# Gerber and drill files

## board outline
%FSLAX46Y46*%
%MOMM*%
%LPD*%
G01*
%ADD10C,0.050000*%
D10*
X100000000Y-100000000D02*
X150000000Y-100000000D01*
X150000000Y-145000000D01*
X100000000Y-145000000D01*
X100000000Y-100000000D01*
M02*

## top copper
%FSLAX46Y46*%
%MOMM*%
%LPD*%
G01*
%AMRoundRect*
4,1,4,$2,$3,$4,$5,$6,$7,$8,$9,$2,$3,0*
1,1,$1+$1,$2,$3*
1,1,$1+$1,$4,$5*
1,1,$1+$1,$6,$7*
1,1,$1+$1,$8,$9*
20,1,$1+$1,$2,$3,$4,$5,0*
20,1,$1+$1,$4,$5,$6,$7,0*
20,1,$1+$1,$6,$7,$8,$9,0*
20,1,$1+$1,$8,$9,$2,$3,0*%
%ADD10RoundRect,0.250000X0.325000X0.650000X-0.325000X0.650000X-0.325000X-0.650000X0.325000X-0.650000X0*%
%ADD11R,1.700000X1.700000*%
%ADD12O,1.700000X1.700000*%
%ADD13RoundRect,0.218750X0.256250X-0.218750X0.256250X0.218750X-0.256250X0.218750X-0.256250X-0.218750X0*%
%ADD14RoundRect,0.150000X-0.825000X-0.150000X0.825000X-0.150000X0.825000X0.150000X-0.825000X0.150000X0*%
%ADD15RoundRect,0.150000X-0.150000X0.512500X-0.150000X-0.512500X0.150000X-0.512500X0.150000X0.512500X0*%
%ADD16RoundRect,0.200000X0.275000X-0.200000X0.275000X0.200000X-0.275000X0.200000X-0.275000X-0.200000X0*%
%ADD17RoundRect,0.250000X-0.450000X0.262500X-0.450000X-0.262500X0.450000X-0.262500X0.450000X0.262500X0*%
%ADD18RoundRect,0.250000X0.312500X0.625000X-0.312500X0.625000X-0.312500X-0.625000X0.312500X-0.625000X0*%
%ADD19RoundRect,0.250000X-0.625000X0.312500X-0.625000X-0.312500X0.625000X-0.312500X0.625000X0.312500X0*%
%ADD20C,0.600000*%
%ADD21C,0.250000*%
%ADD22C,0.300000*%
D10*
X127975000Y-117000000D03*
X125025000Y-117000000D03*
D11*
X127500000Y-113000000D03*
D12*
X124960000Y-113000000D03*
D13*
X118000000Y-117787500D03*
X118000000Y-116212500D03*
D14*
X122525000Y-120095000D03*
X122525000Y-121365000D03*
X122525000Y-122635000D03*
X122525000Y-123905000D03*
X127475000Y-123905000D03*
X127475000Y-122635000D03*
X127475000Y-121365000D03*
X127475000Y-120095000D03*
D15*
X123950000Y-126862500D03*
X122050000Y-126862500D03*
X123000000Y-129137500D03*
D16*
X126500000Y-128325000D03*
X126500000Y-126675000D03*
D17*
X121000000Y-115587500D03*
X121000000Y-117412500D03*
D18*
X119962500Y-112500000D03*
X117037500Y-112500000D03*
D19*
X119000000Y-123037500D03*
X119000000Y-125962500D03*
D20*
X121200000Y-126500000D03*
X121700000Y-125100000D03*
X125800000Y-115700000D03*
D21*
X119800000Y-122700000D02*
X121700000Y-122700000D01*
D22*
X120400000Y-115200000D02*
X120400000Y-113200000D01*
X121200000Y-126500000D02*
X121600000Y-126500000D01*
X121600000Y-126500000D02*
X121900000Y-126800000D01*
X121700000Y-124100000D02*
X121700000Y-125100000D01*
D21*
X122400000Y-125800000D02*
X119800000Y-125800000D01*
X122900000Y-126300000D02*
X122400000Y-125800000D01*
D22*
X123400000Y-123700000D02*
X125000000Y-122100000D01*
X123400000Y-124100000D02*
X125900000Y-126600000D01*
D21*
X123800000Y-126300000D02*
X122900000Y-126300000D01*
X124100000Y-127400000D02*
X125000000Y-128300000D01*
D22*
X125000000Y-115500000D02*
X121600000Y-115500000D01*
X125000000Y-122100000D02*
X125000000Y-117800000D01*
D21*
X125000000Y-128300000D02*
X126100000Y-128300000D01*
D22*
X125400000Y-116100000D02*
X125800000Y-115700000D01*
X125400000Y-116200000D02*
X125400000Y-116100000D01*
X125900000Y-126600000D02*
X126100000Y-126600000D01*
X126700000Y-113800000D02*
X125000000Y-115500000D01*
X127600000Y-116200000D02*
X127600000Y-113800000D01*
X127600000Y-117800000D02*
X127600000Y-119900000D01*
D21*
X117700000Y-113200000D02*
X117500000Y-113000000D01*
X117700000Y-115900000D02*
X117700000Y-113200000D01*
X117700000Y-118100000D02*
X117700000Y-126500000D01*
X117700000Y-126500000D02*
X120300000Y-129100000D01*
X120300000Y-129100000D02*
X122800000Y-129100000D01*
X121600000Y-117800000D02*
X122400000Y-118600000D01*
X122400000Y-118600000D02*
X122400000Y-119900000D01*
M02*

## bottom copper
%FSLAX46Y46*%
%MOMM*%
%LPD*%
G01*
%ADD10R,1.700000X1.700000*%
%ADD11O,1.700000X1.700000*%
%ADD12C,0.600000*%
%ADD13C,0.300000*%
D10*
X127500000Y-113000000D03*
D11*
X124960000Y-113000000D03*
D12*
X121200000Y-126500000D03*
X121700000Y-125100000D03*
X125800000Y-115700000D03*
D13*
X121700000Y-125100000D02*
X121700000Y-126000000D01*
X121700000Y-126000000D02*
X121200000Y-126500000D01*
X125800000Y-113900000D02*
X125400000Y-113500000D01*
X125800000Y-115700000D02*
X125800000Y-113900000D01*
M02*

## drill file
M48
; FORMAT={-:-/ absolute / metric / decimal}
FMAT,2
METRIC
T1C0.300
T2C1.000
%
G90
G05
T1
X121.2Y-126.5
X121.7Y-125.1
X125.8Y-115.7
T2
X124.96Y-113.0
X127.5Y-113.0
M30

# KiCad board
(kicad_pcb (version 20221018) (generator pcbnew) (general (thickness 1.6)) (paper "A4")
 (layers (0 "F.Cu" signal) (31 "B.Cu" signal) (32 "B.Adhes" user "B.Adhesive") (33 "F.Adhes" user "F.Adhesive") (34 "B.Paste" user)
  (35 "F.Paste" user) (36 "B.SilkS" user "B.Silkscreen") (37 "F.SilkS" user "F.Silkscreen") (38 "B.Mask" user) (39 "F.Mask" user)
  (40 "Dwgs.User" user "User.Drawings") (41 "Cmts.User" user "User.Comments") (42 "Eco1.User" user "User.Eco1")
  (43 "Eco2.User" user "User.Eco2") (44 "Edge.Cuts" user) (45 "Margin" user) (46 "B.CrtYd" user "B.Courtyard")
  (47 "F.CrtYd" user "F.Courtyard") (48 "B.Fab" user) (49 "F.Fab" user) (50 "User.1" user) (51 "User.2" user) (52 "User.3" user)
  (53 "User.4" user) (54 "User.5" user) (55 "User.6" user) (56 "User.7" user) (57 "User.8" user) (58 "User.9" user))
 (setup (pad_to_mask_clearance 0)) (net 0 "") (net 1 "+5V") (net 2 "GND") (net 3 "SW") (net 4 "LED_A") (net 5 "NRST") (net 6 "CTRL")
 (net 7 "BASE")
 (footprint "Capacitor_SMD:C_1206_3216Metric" (layer "F.Cu") (at 126.5 117 180)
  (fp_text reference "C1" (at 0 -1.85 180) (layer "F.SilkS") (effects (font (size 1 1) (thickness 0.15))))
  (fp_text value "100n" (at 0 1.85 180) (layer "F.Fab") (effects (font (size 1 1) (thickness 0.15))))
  (pad "1" smd roundrect (at -1.475 0 180) (size 1.15 1.8) (layers "F.Cu" "F.Paste" "F.Mask") (roundrect_rratio 0.217391) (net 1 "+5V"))
  (pad "2" smd roundrect (at 1.475 0 180) (size 1.15 1.8) (layers "F.Cu" "F.Paste" "F.Mask") (roundrect_rratio 0.217391) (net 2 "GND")))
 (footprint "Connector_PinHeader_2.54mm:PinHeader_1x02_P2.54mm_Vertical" (layer "F.Cu") (at 127.5 113 -90)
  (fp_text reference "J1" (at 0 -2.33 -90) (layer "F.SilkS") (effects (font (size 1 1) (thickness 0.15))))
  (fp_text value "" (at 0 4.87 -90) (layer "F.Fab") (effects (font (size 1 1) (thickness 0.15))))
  (pad "1" thru_hole rect (at 0 0 270) (size 1.7 1.7) (drill 1) (layers "*.Cu" "*.Mask") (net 1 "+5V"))
  (pad "2" thru_hole oval (at 0 2.54 270) (size 1.7 1.7) (drill 1) (layers "*.Cu" "*.Mask") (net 2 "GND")))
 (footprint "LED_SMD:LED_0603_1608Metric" (layer "F.Cu") (at 118 117 90)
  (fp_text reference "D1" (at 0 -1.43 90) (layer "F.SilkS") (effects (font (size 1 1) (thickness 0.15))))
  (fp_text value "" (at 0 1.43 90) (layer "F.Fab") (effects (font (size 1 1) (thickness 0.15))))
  (pad "1" smd roundrect (at -0.7875 0 90) (size 0.875 0.95) (layers "F.Cu" "F.Paste" "F.Mask") (roundrect_rratio 0.25) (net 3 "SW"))
  (pad "2" smd roundrect (at 0.7875 0 90) (size 0.875 0.95) (layers "F.Cu" "F.Paste" "F.Mask") (roundrect_rratio 0.25) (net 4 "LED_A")))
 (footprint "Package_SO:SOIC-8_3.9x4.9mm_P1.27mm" (layer "F.Cu") (at 125 122)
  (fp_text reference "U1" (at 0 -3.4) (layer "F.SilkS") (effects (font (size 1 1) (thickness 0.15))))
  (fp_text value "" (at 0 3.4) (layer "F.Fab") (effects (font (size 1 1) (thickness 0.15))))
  (pad "1" smd roundrect (at -2.475 -1.905) (size 1.95 0.6) (layers "F.Cu" "F.Paste" "F.Mask") (roundrect_rratio 0.25) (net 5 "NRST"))
  (pad "2" smd roundrect (at -2.475 -0.635) (size 1.95 0.6) (layers "F.Cu" "F.Paste" "F.Mask") (roundrect_rratio 0.25))
  (pad "3" smd roundrect (at -2.475 0.635) (size 1.95 0.6) (layers "F.Cu" "F.Paste" "F.Mask") (roundrect_rratio 0.25) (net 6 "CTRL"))
  (pad "4" smd roundrect (at -2.475 1.905) (size 1.95 0.6) (layers "F.Cu" "F.Paste" "F.Mask") (roundrect_rratio 0.25) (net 2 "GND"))
  (pad "5" smd roundrect (at 2.475 1.905) (size 1.95 0.6) (layers "F.Cu" "F.Paste" "F.Mask") (roundrect_rratio 0.25))
  (pad "6" smd roundrect (at 2.475 0.635) (size 1.95 0.6) (layers "F.Cu" "F.Paste" "F.Mask") (roundrect_rratio 0.25))
  (pad "7" smd roundrect (at 2.475 -0.635) (size 1.95 0.6) (layers "F.Cu" "F.Paste" "F.Mask") (roundrect_rratio 0.25))
  (pad "8" smd roundrect (at 2.475 -1.905) (size 1.95 0.6) (layers "F.Cu" "F.Paste" "F.Mask") (roundrect_rratio 0.25) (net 1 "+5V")))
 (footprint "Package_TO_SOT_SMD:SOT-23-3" (layer "F.Cu") (at 123 128 -90)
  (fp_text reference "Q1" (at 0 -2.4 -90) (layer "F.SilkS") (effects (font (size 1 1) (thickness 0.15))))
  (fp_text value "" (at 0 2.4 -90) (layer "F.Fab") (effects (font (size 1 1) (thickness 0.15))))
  (pad "1" smd roundrect (at -1.1375 -0.95 270) (size 1.325 0.6) (layers "F.Cu" "F.Paste" "F.Mask") (roundrect_rratio 0.25) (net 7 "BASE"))
  (pad "2" smd roundrect (at -1.1375 0.95 270) (size 1.325 0.6) (layers "F.Cu" "F.Paste" "F.Mask") (roundrect_rratio 0.25) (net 2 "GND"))
  (pad "3" smd roundrect (at 1.1375 0 270) (size 1.325 0.6) (layers "F.Cu" "F.Paste" "F.Mask") (roundrect_rratio 0.25) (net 3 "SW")))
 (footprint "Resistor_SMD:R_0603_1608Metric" (layer "F.Cu") (at 126.5 127.5 90)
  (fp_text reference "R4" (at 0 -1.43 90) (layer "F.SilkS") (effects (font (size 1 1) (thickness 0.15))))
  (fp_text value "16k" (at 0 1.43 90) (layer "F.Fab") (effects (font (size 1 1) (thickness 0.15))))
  (pad "1" smd roundrect (at -0.825 0 90) (size 0.8 0.95) (layers "F.Cu" "F.Paste" "F.Mask") (roundrect_rratio 0.25) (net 7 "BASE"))
  (pad "2" smd roundrect (at 0.825 0 90) (size 0.8 0.95) (layers "F.Cu" "F.Paste" "F.Mask") (roundrect_rratio 0.25) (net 2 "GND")))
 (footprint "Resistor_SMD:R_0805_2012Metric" (layer "F.Cu") (at 121 116.5 -90)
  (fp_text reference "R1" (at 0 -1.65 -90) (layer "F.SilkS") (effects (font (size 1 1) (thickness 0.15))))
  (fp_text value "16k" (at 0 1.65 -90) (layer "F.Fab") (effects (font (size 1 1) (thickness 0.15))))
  (pad "1" smd roundrect (at -0.9125 0 270) (size 1.025 1.4) (layers "F.Cu" "F.Paste" "F.Mask") (roundrect_rratio 0.243902) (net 1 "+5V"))
  (pad "2" smd roundrect (at 0.9125 0 270) (size 1.025 1.4) (layers "F.Cu" "F.Paste" "F.Mask") (roundrect_rratio 0.243902) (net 5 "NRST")))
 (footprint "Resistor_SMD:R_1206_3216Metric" (layer "F.Cu") (at 118.5 112.5 180)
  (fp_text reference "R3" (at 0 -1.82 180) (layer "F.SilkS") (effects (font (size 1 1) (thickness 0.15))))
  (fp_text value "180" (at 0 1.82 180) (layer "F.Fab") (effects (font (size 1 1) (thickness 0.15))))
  (pad "1" smd roundrect (at -1.4625 0 180) (size 1.125 1.75) (layers "F.Cu" "F.Paste" "F.Mask") (roundrect_rratio 0.222222) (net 1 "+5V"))
  (pad "2" smd roundrect (at 1.4625 0 180) (size 1.125 1.75) (layers "F.Cu" "F.Paste" "F.Mask") (roundrect_rratio 0.222222) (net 4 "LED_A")))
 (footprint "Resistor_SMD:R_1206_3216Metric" (layer "F.Cu") (at 119 124.5 -90)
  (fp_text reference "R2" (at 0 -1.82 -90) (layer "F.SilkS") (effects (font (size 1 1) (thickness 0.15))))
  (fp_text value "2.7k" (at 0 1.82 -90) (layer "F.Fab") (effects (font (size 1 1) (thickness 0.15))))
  (pad "1" smd roundrect (at -1.4625 0 270) (size 1.125 1.75) (layers "F.Cu" "F.Paste" "F.Mask") (roundrect_rratio 0.222222) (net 6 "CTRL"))
  (pad "2" smd roundrect (at 1.4625 0 270) (size 1.125 1.75) (layers "F.Cu" "F.Paste" "F.Mask") (roundrect_rratio 0.222222) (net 7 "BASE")))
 (gr_rect (start 100 100) (end 150 145) (stroke (width 0.05) (type default)) (fill none) (layer "Edge.Cuts"))
 (segment (start 119.8 122.7) (end 121.7 122.7) (width 0.25) (layer "F.Cu") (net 6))
 (segment (start 120.4 115.2) (end 120.4 113.2) (width 0.3) (layer "F.Cu") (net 1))
 (segment (start 121.2 126.5) (end 121.6 126.5) (width 0.3) (layer "F.Cu") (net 2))
 (segment (start 121.6 126.5) (end 121.9 126.8) (width 0.3) (layer "F.Cu") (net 2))
 (segment (start 121.7 124.1) (end 121.7 125.1) (width 0.3) (layer "F.Cu") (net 2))
 (segment (start 122.4 125.8) (end 119.8 125.8) (width 0.25) (layer "F.Cu") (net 7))
 (segment (start 122.9 126.3) (end 122.4 125.8) (width 0.25) (layer "F.Cu") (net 7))
 (segment (start 123.4 123.7) (end 125 122.1) (width 0.3) (layer "F.Cu") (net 2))
 (segment (start 123.4 124.1) (end 125.9 126.6) (width 0.3) (layer "F.Cu") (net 2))
 (segment (start 123.8 126.3) (end 122.9 126.3) (width 0.25) (layer "F.Cu") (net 7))
 (segment (start 124.1 127.4) (end 125 128.3) (width 0.25) (layer "F.Cu") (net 7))
 (segment (start 125 115.5) (end 121.6 115.5) (width 0.3) (layer "F.Cu") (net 1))
 (segment (start 125 122.1) (end 125 117.8) (width 0.3) (layer "F.Cu") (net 2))
 (segment (start 125 128.3) (end 126.1 128.3) (width 0.25) (layer "F.Cu") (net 7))
 (segment (start 125.4 116.1) (end 125.8 115.7) (width 0.3) (layer "F.Cu") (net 2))
 (segment (start 125.4 116.2) (end 125.4 116.1) (width 0.3) (layer "F.Cu") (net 2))
 (segment (start 125.9 126.6) (end 126.1 126.6) (width 0.3) (layer "F.Cu") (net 2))
 (segment (start 126.7 113.8) (end 125 115.5) (width 0.3) (layer "F.Cu") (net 1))
 (segment (start 127.6 116.2) (end 127.6 113.8) (width 0.3) (layer "F.Cu") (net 1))
 (segment (start 127.6 117.8) (end 127.6 119.9) (width 0.3) (layer "F.Cu") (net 1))
 (via (at 121.2 126.5) (size 0.6) (drill 0.3) (layers "F.Cu" "B.Cu") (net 2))
 (via (at 121.7 125.1) (size 0.6) (drill 0.3) (layers "F.Cu" "B.Cu") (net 2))
 (via (at 125.8 115.7) (size 0.6) (drill 0.3) (layers "F.Cu" "B.Cu") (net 2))
 (segment (start 117.7 113.2) (end 117.5 113) (width 0.25) (layer "F.Cu") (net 4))
 (segment (start 117.7 115.9) (end 117.7 113.2) (width 0.25) (layer "F.Cu") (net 4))
 (segment (start 117.7 118.1) (end 117.7 126.5) (width 0.25) (layer "F.Cu") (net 3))
 (segment (start 117.7 126.5) (end 120.3 129.1) (width 0.25) (layer "F.Cu") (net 3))
 (segment (start 120.3 129.1) (end 122.8 129.1) (width 0.25) (layer "F.Cu") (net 3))
 (segment (start 121.6 117.8) (end 122.4 118.6) (width 0.25) (layer "F.Cu") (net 5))
 (segment (start 121.7 125.1) (end 121.7 126) (width 0.3) (layer "B.Cu") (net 2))
 (segment (start 121.7 126) (end 121.2 126.5) (width 0.3) (layer "B.Cu") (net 2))
 (segment (start 122.4 118.6) (end 122.4 119.9) (width 0.25) (layer "F.Cu") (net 5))
 (segment (start 125.8 113.9) (end 125.4 113.5) (width 0.3) (layer "B.Cu") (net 2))
 (segment (start 125.8 115.7) (end 125.8 113.9) (width 0.3) (layer "B.Cu") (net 2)))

